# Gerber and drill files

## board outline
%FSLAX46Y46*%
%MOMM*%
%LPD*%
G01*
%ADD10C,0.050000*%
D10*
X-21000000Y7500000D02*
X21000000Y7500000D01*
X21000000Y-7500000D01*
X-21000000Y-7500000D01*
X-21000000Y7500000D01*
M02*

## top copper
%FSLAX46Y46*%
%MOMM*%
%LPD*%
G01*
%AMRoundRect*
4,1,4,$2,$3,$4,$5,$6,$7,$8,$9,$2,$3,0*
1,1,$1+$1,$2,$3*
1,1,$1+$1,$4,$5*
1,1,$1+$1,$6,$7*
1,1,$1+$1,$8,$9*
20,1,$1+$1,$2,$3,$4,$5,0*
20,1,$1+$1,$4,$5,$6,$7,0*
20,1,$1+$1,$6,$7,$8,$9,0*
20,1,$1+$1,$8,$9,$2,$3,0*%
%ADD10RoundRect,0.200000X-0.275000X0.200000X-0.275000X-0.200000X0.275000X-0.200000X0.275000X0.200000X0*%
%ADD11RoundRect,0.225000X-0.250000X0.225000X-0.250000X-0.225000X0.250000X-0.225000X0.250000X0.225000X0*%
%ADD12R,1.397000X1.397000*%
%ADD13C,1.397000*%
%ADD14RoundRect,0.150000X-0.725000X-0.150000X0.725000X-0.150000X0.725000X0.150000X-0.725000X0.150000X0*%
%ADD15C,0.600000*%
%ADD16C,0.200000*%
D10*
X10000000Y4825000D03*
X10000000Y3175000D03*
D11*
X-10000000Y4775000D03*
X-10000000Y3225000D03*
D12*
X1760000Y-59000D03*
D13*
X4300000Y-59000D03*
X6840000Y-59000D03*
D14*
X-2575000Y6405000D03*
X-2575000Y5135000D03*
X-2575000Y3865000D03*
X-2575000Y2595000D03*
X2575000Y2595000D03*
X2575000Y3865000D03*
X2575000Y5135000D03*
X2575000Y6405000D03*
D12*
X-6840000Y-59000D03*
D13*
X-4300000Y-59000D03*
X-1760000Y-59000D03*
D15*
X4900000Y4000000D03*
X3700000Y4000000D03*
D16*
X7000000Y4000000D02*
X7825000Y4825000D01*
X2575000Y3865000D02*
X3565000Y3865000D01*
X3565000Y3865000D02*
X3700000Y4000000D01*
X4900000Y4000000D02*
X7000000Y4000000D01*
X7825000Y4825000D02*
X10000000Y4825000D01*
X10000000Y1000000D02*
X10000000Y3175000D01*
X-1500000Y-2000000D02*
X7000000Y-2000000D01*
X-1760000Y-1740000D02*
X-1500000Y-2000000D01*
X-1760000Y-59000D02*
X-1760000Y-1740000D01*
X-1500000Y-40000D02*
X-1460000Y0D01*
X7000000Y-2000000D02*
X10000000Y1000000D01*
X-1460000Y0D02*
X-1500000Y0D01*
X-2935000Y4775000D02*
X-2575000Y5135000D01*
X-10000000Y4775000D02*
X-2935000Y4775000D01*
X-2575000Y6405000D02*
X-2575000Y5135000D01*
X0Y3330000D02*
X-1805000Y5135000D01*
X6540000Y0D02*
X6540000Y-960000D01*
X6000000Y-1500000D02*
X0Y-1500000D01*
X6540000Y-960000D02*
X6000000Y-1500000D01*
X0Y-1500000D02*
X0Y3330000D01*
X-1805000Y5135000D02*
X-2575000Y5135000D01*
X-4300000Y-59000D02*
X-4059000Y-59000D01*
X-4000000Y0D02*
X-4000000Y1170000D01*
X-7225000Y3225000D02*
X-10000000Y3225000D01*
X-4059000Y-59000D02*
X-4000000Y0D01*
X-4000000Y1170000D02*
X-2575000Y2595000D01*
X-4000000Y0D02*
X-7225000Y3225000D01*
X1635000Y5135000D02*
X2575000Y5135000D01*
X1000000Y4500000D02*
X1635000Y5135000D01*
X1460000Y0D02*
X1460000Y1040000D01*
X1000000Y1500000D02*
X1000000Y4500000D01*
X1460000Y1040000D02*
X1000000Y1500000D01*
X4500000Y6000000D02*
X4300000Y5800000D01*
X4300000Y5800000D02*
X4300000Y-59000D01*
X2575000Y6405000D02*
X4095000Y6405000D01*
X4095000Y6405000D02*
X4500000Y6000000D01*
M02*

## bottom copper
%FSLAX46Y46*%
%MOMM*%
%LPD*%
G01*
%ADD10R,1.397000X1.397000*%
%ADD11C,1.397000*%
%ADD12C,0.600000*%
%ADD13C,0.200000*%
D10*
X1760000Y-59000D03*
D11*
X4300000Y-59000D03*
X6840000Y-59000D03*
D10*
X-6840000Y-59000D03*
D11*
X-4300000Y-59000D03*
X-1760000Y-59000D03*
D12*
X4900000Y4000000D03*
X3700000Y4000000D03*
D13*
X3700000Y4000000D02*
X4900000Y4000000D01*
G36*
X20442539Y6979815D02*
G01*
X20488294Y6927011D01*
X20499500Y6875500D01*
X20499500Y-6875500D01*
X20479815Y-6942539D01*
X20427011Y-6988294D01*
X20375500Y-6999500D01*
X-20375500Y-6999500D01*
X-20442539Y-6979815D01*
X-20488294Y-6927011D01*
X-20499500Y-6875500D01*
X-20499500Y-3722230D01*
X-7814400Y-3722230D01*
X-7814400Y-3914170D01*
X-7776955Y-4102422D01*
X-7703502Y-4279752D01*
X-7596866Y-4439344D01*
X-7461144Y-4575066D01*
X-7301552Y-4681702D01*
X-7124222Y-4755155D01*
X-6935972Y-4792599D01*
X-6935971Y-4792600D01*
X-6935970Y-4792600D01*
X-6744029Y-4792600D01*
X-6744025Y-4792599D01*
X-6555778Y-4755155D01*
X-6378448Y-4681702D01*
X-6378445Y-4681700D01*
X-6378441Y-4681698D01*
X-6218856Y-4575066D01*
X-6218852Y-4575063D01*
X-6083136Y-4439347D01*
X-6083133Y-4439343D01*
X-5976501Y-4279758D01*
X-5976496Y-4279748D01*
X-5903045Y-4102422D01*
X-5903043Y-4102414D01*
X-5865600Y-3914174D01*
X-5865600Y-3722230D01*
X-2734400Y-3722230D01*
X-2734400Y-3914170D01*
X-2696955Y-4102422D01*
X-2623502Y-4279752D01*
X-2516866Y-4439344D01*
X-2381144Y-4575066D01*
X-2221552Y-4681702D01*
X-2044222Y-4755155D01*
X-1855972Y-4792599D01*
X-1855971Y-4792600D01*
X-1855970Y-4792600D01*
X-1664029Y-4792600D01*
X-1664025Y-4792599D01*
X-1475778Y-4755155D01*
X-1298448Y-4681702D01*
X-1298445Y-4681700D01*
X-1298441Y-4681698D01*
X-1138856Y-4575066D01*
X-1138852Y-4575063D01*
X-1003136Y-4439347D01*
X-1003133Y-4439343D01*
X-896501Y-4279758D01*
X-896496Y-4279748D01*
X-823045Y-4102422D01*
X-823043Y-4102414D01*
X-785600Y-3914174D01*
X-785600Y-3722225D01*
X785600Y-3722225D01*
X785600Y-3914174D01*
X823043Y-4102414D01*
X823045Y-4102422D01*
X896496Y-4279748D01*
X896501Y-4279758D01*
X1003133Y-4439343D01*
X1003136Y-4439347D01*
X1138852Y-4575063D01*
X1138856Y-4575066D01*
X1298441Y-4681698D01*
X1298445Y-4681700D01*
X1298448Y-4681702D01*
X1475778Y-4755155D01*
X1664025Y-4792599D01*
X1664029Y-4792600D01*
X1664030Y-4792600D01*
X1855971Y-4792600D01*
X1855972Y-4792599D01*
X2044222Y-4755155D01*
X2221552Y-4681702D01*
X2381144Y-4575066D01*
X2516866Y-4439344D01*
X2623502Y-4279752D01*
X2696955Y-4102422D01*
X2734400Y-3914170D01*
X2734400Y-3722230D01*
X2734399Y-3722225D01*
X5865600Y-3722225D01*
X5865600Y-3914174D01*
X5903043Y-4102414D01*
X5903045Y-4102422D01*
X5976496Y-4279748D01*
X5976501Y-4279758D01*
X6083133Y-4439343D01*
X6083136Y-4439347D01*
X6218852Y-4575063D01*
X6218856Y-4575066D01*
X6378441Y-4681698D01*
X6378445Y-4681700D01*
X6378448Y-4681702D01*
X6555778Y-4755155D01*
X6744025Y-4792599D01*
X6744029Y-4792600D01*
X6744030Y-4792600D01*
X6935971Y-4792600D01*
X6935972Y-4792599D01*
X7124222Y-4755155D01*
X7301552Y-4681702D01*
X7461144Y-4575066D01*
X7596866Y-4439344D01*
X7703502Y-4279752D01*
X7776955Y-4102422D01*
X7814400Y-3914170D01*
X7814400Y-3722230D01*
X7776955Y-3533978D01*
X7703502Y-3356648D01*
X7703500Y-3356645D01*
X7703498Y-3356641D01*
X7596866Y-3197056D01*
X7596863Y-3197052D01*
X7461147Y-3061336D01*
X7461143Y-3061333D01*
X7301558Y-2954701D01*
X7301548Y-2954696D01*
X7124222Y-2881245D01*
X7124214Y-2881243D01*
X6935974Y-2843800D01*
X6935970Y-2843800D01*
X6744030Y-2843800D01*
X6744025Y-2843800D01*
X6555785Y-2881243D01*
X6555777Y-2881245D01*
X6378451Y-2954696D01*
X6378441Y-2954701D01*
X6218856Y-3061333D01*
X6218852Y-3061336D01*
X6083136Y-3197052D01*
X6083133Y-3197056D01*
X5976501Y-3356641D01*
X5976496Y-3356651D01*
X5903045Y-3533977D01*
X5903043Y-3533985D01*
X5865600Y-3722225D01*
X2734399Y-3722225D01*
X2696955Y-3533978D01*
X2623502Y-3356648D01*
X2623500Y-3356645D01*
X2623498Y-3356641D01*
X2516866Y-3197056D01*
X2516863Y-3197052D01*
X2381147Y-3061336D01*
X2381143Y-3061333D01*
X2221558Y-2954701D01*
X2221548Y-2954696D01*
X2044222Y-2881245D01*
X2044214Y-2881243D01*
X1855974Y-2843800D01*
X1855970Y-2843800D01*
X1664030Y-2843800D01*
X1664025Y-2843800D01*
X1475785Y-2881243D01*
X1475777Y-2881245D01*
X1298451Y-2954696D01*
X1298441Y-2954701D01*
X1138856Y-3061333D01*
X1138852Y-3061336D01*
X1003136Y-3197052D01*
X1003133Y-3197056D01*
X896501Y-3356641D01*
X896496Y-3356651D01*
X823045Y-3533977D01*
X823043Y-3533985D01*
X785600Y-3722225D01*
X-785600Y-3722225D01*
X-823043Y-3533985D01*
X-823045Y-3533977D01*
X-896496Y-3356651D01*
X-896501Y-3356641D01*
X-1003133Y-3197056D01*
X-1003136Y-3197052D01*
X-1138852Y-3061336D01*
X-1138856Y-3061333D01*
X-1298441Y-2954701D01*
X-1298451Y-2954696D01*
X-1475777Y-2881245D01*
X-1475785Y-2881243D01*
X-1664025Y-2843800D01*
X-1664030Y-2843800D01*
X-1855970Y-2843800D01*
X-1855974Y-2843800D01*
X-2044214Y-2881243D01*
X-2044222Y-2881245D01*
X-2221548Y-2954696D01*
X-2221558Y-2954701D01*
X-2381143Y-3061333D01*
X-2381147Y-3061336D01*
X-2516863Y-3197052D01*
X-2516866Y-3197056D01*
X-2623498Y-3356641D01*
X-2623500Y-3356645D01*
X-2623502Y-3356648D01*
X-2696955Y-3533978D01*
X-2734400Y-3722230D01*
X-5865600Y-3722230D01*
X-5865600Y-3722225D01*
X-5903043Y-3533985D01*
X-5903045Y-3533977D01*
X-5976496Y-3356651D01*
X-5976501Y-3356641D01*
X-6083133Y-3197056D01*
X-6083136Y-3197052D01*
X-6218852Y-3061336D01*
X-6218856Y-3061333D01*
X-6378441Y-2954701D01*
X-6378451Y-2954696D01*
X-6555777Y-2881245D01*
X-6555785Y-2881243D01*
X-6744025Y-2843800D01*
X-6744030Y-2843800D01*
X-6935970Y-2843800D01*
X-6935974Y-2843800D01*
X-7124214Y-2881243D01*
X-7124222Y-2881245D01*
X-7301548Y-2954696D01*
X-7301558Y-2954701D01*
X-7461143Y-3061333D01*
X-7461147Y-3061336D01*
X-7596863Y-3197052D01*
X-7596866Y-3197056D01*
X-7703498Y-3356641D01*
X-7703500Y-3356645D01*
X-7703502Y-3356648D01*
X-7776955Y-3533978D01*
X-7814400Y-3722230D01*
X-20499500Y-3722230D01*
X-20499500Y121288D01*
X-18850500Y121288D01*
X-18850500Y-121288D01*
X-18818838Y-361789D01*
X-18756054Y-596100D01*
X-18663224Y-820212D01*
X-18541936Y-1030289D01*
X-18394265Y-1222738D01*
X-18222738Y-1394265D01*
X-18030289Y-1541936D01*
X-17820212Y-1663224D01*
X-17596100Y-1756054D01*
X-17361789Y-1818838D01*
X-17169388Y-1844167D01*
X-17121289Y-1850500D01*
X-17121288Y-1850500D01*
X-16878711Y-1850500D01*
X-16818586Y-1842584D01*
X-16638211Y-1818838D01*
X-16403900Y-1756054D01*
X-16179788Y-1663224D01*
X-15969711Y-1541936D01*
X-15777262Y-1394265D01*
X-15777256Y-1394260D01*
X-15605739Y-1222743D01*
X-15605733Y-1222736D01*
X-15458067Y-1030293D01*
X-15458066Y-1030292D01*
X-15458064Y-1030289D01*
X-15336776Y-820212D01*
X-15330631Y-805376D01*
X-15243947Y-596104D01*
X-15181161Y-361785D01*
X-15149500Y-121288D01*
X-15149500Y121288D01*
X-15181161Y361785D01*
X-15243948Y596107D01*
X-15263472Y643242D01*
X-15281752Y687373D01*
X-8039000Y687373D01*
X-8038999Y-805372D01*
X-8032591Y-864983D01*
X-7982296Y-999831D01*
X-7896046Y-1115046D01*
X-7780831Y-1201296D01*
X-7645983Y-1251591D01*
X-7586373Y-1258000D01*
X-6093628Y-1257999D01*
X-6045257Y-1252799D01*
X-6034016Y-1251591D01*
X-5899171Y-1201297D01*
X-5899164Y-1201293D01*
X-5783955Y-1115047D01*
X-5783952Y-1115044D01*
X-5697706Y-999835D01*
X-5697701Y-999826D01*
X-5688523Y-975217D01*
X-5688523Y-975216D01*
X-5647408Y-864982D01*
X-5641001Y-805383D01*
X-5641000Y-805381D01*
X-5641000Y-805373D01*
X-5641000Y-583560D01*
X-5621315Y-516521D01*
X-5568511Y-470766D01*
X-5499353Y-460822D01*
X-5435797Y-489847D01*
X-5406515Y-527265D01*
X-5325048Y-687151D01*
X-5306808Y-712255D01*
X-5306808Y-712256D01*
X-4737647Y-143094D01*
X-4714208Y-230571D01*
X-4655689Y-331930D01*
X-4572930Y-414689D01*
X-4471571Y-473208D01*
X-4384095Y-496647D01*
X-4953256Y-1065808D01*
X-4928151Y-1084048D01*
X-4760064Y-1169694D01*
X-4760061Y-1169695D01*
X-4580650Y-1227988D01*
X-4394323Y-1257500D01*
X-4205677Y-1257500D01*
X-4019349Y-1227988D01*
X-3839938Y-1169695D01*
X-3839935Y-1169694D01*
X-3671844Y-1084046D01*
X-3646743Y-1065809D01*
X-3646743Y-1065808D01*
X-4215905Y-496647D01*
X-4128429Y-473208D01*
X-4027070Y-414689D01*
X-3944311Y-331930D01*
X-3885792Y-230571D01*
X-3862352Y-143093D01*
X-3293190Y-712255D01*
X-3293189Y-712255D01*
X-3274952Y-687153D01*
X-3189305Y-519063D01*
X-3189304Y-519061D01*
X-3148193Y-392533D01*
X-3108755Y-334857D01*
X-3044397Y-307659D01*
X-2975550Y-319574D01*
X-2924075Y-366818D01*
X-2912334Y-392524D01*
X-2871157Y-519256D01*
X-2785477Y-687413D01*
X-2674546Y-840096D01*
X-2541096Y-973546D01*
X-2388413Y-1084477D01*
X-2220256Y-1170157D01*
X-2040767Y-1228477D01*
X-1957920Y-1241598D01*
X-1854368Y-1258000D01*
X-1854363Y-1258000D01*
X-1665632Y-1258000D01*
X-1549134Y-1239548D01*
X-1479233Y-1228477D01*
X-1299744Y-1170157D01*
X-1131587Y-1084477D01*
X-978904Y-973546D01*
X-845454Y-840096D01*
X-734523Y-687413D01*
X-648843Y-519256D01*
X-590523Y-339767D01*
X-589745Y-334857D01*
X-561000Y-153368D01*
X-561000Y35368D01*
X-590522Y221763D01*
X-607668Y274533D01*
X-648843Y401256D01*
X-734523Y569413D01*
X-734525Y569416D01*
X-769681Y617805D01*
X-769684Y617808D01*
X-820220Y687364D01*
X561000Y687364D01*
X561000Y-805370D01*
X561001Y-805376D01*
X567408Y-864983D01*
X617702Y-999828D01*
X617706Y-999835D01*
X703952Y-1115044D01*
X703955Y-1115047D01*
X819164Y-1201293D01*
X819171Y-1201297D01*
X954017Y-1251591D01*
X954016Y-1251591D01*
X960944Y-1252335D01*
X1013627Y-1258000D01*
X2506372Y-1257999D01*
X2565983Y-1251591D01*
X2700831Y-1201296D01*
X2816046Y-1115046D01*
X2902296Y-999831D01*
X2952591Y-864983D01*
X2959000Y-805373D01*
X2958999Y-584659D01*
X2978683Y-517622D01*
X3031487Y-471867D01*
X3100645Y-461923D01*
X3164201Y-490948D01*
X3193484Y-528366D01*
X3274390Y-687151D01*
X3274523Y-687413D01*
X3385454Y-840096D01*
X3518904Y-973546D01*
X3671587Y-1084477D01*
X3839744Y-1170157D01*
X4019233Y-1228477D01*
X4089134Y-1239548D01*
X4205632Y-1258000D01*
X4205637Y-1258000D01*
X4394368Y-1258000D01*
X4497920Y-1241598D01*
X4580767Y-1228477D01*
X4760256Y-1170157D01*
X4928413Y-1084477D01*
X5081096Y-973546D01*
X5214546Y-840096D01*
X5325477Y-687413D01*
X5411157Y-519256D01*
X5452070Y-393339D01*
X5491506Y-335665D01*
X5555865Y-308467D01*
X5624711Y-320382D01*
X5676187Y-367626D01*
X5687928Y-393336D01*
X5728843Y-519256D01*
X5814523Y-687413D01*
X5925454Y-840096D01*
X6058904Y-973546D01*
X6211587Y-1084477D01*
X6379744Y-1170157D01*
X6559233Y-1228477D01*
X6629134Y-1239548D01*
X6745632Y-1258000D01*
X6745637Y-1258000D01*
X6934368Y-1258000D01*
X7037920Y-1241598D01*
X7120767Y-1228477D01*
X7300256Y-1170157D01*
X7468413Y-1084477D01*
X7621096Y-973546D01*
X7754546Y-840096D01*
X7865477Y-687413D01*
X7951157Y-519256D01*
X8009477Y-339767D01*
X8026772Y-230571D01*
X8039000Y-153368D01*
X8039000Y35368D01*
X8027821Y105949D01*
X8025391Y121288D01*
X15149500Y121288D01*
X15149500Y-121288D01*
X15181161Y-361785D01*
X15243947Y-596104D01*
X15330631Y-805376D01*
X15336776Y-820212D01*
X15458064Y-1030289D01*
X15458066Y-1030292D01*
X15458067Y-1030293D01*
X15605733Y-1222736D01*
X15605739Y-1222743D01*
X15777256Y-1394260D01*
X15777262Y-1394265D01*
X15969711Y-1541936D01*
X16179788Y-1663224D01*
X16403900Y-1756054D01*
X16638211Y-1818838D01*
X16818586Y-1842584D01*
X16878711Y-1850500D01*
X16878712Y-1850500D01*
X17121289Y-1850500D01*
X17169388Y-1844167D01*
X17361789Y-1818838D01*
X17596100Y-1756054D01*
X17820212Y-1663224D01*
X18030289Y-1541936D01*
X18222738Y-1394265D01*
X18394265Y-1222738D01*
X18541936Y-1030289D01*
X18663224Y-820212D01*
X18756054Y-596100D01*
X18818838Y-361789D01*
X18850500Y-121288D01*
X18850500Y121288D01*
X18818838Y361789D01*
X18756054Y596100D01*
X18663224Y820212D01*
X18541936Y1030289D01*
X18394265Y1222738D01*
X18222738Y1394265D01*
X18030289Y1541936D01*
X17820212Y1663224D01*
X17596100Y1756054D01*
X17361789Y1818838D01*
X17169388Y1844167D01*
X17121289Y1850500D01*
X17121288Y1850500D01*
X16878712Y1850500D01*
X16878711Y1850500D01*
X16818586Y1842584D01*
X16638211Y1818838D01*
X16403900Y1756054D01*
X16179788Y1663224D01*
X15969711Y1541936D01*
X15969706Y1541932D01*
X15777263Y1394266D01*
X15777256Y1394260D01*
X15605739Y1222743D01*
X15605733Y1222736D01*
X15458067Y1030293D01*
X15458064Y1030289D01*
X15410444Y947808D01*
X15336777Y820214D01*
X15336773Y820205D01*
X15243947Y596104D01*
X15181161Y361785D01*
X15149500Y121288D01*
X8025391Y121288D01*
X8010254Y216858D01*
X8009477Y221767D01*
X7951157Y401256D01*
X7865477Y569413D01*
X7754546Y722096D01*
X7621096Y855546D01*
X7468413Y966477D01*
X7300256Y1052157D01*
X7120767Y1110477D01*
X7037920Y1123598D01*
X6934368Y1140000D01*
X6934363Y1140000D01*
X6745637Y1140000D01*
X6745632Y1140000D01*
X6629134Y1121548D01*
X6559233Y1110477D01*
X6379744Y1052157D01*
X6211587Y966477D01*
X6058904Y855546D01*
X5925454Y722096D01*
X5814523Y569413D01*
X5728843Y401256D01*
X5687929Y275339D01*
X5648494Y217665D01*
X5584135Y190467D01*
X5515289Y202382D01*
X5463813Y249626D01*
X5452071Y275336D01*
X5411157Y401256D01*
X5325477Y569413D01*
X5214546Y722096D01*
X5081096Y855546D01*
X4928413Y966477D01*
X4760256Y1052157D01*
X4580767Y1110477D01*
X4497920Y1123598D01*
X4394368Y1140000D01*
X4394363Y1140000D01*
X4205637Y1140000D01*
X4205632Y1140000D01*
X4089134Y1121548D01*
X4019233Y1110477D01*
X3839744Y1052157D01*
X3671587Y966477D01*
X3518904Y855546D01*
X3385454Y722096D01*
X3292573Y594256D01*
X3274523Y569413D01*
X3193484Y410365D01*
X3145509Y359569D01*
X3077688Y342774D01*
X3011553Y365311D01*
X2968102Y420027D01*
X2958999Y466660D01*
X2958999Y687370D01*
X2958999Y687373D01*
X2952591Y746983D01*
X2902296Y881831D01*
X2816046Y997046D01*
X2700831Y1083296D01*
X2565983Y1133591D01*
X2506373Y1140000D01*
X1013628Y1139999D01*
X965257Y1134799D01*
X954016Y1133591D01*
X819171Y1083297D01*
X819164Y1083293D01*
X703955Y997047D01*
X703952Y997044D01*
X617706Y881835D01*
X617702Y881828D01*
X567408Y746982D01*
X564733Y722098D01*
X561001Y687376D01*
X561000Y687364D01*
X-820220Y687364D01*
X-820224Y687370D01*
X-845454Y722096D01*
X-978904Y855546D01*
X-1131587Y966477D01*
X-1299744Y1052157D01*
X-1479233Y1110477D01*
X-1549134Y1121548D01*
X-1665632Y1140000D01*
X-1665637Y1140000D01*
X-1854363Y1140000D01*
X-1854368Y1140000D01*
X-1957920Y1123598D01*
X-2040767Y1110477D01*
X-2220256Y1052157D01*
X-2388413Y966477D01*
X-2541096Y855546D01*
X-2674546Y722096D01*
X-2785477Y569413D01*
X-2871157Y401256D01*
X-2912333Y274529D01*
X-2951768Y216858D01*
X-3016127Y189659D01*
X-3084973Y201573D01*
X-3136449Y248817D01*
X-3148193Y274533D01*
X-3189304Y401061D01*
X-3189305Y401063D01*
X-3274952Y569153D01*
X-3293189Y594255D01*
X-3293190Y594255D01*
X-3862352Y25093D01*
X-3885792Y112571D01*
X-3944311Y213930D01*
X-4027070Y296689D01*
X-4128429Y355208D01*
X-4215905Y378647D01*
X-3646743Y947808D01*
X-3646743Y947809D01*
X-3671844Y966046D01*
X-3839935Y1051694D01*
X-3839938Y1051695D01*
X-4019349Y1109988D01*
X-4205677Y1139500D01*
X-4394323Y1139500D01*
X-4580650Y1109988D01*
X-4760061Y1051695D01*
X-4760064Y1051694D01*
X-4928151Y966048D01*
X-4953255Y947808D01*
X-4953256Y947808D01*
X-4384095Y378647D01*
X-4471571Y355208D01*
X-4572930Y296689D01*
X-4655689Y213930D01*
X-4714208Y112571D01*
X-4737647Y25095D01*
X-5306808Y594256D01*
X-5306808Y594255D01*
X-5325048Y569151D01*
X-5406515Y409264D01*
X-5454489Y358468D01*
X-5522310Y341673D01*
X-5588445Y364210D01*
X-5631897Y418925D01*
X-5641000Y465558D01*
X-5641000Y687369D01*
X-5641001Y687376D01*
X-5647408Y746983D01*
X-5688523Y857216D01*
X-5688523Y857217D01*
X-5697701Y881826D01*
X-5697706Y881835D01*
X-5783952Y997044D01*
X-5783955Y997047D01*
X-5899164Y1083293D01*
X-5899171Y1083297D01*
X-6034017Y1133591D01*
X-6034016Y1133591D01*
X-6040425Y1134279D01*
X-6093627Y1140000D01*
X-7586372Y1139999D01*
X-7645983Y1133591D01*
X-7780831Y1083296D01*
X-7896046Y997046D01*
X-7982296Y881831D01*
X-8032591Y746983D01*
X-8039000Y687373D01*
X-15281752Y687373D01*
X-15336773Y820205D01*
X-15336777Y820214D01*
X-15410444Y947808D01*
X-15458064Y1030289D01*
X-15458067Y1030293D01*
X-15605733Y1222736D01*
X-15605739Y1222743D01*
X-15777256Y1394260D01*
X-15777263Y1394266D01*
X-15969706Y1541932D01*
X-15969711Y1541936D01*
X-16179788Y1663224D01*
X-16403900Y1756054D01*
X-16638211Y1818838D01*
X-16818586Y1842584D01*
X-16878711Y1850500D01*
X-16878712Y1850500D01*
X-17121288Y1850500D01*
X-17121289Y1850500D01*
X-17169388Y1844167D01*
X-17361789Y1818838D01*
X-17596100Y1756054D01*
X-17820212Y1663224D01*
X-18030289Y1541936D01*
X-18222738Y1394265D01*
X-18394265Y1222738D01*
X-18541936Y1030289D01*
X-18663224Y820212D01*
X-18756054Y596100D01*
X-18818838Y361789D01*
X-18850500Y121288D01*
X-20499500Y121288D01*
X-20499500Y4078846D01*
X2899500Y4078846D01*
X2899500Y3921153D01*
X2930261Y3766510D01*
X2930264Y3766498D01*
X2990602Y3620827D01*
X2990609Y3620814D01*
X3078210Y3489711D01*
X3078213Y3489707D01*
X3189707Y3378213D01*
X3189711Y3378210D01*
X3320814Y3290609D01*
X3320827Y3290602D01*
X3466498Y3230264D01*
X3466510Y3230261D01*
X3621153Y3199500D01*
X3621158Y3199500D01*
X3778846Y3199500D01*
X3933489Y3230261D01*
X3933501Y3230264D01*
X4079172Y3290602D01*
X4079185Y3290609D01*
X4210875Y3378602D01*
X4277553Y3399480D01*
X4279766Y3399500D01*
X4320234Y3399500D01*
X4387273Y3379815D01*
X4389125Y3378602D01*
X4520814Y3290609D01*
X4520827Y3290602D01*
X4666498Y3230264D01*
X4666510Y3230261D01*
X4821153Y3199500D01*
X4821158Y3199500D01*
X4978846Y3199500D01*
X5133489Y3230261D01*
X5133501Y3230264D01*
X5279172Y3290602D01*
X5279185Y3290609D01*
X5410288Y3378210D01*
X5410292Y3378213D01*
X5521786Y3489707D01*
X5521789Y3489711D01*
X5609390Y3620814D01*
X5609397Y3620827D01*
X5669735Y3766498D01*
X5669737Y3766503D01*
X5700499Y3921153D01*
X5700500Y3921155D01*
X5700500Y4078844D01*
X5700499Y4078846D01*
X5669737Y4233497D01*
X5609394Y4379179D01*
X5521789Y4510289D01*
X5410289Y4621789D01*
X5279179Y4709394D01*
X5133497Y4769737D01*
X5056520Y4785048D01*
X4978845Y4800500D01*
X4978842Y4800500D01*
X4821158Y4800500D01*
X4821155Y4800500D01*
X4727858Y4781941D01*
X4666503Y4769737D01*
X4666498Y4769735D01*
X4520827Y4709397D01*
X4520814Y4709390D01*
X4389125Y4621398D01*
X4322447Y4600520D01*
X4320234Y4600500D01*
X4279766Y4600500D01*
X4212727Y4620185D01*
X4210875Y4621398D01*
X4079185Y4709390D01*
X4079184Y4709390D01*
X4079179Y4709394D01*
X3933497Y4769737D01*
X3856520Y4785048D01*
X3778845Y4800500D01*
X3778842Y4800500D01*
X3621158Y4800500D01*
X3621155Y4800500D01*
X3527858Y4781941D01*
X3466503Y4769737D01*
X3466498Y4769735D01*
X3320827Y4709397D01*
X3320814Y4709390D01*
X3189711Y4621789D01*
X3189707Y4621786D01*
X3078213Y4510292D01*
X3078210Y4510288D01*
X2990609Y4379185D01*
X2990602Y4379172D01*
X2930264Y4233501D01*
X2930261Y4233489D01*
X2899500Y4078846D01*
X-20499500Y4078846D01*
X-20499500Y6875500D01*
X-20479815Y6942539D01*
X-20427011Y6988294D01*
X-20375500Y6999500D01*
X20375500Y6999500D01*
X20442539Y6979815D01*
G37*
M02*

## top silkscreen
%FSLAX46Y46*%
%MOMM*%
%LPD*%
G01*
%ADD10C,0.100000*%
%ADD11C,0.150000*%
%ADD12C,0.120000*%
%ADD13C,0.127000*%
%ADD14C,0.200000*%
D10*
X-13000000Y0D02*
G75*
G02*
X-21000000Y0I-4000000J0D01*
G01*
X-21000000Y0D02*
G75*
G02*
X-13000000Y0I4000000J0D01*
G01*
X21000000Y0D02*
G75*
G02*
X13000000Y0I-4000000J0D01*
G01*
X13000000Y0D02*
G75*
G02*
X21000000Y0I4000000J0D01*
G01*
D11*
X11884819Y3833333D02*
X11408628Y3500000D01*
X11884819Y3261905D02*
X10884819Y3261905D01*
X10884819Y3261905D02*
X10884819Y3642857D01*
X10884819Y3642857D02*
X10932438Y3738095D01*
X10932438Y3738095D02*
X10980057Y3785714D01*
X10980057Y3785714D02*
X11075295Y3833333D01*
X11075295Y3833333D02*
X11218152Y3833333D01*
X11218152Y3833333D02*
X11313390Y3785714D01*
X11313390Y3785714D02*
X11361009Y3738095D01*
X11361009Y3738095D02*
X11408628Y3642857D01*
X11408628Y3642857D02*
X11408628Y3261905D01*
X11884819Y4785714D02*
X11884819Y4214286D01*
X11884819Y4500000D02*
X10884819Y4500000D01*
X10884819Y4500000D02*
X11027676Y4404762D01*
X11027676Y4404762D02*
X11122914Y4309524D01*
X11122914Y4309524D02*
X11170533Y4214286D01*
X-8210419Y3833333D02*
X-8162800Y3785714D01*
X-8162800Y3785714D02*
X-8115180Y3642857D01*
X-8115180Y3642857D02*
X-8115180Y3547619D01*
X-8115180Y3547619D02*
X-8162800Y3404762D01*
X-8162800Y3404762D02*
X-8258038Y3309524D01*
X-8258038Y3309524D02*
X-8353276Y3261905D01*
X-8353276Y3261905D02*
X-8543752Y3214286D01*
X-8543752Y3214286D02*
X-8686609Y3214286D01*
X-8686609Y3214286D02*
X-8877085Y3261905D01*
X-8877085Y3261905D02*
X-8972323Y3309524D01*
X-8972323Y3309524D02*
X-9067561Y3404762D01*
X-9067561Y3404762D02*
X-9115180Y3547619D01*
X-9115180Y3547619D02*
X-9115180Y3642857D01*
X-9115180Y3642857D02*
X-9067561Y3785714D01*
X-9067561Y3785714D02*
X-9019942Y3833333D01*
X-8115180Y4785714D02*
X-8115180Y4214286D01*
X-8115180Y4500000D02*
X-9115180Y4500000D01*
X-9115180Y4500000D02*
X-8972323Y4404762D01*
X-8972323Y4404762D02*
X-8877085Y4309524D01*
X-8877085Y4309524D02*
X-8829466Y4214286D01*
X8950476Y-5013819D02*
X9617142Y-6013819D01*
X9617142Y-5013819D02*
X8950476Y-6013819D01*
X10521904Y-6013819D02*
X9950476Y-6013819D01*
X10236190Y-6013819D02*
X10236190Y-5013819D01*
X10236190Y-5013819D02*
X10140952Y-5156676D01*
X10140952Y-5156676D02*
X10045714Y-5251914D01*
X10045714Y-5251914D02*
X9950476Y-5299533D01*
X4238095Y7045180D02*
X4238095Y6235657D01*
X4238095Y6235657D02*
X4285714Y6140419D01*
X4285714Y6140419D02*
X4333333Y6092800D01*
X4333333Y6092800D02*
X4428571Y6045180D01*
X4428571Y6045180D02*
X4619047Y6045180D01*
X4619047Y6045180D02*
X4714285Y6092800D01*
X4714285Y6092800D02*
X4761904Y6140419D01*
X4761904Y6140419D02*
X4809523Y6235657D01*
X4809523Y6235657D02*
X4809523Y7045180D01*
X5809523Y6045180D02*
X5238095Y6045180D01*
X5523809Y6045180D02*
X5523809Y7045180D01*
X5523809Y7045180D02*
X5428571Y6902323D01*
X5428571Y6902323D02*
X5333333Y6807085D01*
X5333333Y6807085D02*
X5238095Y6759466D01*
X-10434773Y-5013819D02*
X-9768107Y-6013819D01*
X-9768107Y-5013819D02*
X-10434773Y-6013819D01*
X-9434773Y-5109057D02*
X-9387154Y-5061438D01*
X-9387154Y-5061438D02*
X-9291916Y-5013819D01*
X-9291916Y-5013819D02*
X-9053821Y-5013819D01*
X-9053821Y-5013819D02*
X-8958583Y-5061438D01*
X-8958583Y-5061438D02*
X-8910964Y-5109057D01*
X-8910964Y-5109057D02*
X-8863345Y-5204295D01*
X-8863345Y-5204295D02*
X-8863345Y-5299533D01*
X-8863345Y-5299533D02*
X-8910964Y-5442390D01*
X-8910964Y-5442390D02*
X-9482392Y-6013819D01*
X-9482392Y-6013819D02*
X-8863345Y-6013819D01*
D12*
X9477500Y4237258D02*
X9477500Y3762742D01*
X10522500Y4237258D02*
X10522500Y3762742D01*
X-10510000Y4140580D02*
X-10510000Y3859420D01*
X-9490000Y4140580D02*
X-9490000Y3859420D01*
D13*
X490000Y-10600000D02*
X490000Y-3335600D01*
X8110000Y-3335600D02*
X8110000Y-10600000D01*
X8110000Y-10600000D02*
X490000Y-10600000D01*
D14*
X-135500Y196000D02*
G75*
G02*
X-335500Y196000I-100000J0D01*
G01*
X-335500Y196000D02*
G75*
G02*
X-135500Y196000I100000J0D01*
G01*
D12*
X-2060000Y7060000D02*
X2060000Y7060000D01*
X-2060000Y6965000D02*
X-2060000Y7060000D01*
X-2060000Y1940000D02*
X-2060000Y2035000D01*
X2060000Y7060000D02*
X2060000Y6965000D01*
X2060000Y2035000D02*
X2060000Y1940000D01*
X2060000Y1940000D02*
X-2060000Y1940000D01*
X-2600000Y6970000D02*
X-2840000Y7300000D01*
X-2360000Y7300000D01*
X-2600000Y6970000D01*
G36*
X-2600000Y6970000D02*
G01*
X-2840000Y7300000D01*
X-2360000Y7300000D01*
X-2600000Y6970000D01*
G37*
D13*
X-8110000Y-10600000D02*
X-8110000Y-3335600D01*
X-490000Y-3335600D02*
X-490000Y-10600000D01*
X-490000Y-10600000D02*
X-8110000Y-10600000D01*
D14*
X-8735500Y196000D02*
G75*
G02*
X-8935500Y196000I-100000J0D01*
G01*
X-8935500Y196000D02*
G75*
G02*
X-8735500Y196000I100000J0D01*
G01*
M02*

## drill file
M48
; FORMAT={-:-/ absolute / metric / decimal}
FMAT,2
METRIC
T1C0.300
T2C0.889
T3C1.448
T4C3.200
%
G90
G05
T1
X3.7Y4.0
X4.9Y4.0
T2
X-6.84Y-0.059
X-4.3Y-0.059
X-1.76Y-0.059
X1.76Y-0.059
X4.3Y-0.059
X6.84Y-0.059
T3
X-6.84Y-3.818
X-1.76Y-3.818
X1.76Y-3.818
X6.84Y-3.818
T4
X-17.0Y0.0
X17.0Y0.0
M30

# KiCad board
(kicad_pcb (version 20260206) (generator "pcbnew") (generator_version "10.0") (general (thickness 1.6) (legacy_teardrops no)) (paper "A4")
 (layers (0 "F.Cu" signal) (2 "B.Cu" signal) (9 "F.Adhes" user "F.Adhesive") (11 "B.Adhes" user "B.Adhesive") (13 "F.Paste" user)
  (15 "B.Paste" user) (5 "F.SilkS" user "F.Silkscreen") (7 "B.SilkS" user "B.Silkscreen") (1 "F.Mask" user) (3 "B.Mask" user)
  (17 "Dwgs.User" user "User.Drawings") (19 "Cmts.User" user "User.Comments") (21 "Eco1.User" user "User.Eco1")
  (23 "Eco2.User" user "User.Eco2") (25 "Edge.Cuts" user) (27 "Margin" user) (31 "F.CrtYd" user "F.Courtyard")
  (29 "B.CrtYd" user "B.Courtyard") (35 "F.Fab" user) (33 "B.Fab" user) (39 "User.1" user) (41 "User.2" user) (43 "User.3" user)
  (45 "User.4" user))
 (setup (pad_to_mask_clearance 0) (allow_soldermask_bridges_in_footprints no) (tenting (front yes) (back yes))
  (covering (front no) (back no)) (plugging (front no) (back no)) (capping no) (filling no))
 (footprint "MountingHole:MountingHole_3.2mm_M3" (layer "F.Cu") (at 17 0)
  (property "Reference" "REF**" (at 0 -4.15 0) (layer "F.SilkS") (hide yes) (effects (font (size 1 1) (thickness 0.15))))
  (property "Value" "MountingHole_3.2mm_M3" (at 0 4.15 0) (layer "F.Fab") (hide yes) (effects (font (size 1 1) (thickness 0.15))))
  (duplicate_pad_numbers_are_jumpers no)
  (pad "" np_thru_hole circle (at 0 0) (size 3.2 3.2) (drill 3.2) (layers "*.Cu" "*.Mask")))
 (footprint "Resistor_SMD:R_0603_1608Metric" (layer "F.Cu") (at 10 -4 -90)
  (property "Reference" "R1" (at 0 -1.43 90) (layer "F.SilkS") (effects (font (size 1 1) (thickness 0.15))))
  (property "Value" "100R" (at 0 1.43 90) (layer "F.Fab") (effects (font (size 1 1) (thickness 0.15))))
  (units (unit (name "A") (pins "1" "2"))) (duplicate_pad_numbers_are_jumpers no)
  (fp_line (start -0.237258 0.5225) (end 0.237258 0.5225) (stroke (width 0.12) (type solid)) (layer "F.SilkS"))
  (fp_line (start -0.237258 -0.5225) (end 0.237258 -0.5225) (stroke (width 0.12) (type solid)) (layer "F.SilkS"))
  (pad "1" smd roundrect (at -0.825 0 270) (size 0.8 0.95) (layers "F.Cu" "F.Mask" "F.Paste") (roundrect_rratio 0.25) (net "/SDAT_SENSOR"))
  (pad "2" smd roundrect (at 0.825 0 270) (size 0.8 0.95) (layers "F.Cu" "F.Mask" "F.Paste") (roundrect_rratio 0.25) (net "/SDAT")))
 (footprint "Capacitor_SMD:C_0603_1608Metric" (layer "F.Cu") (at -10 -4 -90)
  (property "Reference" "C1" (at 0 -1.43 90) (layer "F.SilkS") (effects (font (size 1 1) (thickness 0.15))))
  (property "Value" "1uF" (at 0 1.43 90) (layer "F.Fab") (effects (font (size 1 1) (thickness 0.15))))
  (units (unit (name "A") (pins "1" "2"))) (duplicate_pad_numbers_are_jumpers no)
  (fp_line (start -0.14058 0.51) (end 0.14058 0.51) (stroke (width 0.12) (type solid)) (layer "F.SilkS"))
  (fp_line (start -0.14058 -0.51) (end 0.14058 -0.51) (stroke (width 0.12) (type solid)) (layer "F.SilkS"))
  (pad "1" smd roundrect (at -0.775 0 270) (size 0.9 0.95) (layers "F.Cu" "F.Mask" "F.Paste") (roundrect_rratio 0.25) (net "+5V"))
  (pad "2" smd roundrect (at 0.775 0 270) (size 0.9 0.95) (layers "F.Cu" "F.Mask" "F.Paste") (roundrect_rratio 0.25) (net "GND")))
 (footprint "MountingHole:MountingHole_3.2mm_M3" (layer "F.Cu") (at -17 0)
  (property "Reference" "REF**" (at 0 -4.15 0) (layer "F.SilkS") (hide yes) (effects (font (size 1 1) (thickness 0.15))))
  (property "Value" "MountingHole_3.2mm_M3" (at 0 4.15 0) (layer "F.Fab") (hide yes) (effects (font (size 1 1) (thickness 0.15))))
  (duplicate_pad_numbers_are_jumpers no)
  (pad "" np_thru_hole circle (at 0 0) (size 3.2 3.2) (drill 3.2) (layers "*.Cu" "*.Mask")))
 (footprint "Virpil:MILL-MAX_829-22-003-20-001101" (layer "F.Cu") (at 4.3 0.059)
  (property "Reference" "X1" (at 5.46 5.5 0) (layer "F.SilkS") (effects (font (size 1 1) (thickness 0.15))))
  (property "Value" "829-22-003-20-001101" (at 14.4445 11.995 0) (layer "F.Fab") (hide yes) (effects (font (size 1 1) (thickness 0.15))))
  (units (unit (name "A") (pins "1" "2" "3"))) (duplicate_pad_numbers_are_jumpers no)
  (fp_line (start -3.81 10.541) (end -3.81 3.2766) (stroke (width 0.127) (type solid)) (layer "F.SilkS"))
  (fp_line (start 3.81 3.2766) (end 3.81 10.541) (stroke (width 0.127) (type solid)) (layer "F.SilkS"))
  (fp_line (start 3.81 10.541) (end -3.81 10.541) (stroke (width 0.127) (type solid)) (layer "F.SilkS"))
  (fp_circle (center -4.5355 -0.255) (end -4.4355 -0.255) (stroke (width 0.2) (type solid)) (fill no) (layer "F.SilkS"))
  (pad "" np_thru_hole circle (at -2.54 3.7592) (size 1.4478 1.4478) (drill 1.4478) (layers "*.Cu" "*.Mask"))
  (pad "" np_thru_hole circle (at 2.54 3.7592) (size 1.4478 1.4478) (drill 1.4478) (layers "*.Cu" "*.Mask"))
  (pad "1" thru_hole rect (at -2.54 0) (size 1.397 1.397) (drill 0.889) (layers "*.Cu" "*.Mask") (remove_unused_layers no) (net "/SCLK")
   (solder_mask_margin 0.102))
  (pad "2" thru_hole circle (at 0 0) (size 1.397 1.397) (drill 0.889) (layers "*.Cu" "*.Mask") (remove_unused_layers no) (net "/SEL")
   (solder_mask_margin 0.102))
  (pad "3" thru_hole circle (at 2.54 0) (size 1.397 1.397) (drill 0.889) (layers "*.Cu" "*.Mask") (remove_unused_layers no) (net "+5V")
   (solder_mask_margin 0.102)))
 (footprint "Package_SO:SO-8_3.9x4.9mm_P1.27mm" (layer "F.Cu") (at 0 -4.5)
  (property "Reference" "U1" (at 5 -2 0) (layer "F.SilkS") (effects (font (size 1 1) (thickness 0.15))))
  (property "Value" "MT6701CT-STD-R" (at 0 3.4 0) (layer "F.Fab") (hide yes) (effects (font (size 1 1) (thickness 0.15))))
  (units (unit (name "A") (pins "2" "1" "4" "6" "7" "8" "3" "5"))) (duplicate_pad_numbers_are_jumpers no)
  (fp_line (start -2.06 -2.56) (end 2.06 -2.56) (stroke (width 0.12) (type solid)) (layer "F.SilkS"))
  (fp_line (start -2.06 -2.465) (end -2.06 -2.56) (stroke (width 0.12) (type solid)) (layer "F.SilkS"))
  (fp_line (start -2.06 2.56) (end -2.06 2.465) (stroke (width 0.12) (type solid)) (layer "F.SilkS"))
  (fp_line (start 2.06 -2.56) (end 2.06 -2.465) (stroke (width 0.12) (type solid)) (layer "F.SilkS"))
  (fp_line (start 2.06 2.465) (end 2.06 2.56) (stroke (width 0.12) (type solid)) (layer "F.SilkS"))
  (fp_line (start 2.06 2.56) (end -2.06 2.56) (stroke (width 0.12) (type solid)) (layer "F.SilkS"))
  (fp_poly (pts (xy -2.6 -2.47) (xy -2.84 -2.8) (xy -2.36 -2.8)) (stroke (width 0.12) (type solid)) (fill yes) (layer "F.SilkS"))
  (pad "1" smd roundrect (at -2.575 -1.905) (size 1.75 0.6) (layers "F.Cu" "F.Mask" "F.Paste") (roundrect_rratio 0.25) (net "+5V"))
  (pad "2" smd roundrect (at -2.575 -0.635) (size 1.75 0.6) (layers "F.Cu" "F.Mask" "F.Paste") (roundrect_rratio 0.25) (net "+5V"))
  (pad "3" smd roundrect (at -2.575 0.635) (size 1.75 0.6) (layers "F.Cu" "F.Mask" "F.Paste") (roundrect_rratio 0.25)
   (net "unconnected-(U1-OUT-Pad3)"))
  (pad "4" smd roundrect (at -2.575 1.905) (size 1.75 0.6) (layers "F.Cu" "F.Mask" "F.Paste") (roundrect_rratio 0.25) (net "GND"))
  (pad "5" smd roundrect (at 2.575 1.905) (size 1.75 0.6) (layers "F.Cu" "F.Mask" "F.Paste") (roundrect_rratio 0.25)
   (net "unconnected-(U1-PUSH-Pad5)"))
  (pad "6" smd roundrect (at 2.575 0.635) (size 1.75 0.6) (layers "F.Cu" "F.Mask" "F.Paste") (roundrect_rratio 0.25) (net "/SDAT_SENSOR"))
  (pad "7" smd roundrect (at 2.575 -0.635) (size 1.75 0.6) (layers "F.Cu" "F.Mask" "F.Paste") (roundrect_rratio 0.25) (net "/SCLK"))
  (pad "8" smd roundrect (at 2.575 -1.905) (size 1.75 0.6) (layers "F.Cu" "F.Mask" "F.Paste") (roundrect_rratio 0.25) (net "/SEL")))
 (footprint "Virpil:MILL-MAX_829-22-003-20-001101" (layer "F.Cu") (at -4.3 0.059)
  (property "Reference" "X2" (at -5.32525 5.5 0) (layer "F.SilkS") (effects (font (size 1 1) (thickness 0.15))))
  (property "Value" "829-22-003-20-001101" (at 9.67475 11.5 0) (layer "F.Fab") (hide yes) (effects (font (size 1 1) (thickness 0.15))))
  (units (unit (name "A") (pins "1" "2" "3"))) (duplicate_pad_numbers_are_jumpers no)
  (fp_line (start -3.81 10.541) (end -3.81 3.2766) (stroke (width 0.127) (type solid)) (layer "F.SilkS"))
  (fp_line (start 3.81 3.2766) (end 3.81 10.541) (stroke (width 0.127) (type solid)) (layer "F.SilkS"))
  (fp_line (start 3.81 10.541) (end -3.81 10.541) (stroke (width 0.127) (type solid)) (layer "F.SilkS"))
  (fp_circle (center -4.5355 -0.255) (end -4.4355 -0.255) (stroke (width 0.2) (type solid)) (fill no) (layer "F.SilkS"))
  (pad "" np_thru_hole circle (at -2.54 3.7592) (size 1.4478 1.4478) (drill 1.4478) (layers "*.Cu" "*.Mask"))
  (pad "" np_thru_hole circle (at 2.54 3.7592) (size 1.4478 1.4478) (drill 1.4478) (layers "*.Cu" "*.Mask"))
  (pad "1" thru_hole rect (at -2.54 0) (size 1.397 1.397) (drill 0.889) (layers "*.Cu" "*.Mask") (remove_unused_layers no) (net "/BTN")
   (solder_mask_margin 0.102))
  (pad "2" thru_hole circle (at 0 0) (size 1.397 1.397) (drill 0.889) (layers "*.Cu" "*.Mask") (remove_unused_layers no) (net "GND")
   (solder_mask_margin 0.102))
  (pad "3" thru_hole circle (at 2.54 0) (size 1.397 1.397) (drill 0.889) (layers "*.Cu" "*.Mask") (remove_unused_layers no) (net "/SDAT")
   (solder_mask_margin 0.102)))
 (gr_circle (center -17 0) (end -13 0) (stroke (width 0.1) (type default)) (fill no) (layer "F.SilkS"))
 (gr_circle (center 17 0) (end 21 0) (stroke (width 0.1) (type default)) (fill no) (layer "F.SilkS"))
 (gr_rect (start -21 -7.5) (end 21 7.5) (stroke (width 0.05) (type default)) (fill no) (layer "Edge.Cuts"))
 (segment (start 7 -4) (end 7.825 -4.825) (width 0.2) (layer "F.Cu") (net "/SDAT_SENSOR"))
 (segment (start 2.575 -3.865) (end 3.565 -3.865) (width 0.2) (layer "F.Cu") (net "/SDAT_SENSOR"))
 (segment (start 3.565 -3.865) (end 3.7 -4) (width 0.2) (layer "F.Cu") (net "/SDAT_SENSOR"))
 (segment (start 4.9 -4) (end 7 -4) (width 0.2) (layer "F.Cu") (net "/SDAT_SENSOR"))
 (segment (start 7.825 -4.825) (end 10 -4.825) (width 0.2) (layer "F.Cu") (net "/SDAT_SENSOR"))
 (via (at 4.9 -4) (size 0.6) (drill 0.3) (layers "F.Cu" "B.Cu") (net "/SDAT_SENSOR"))
 (via (at 3.7 -4) (size 0.6) (drill 0.3) (layers "F.Cu" "B.Cu") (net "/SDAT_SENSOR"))
 (segment (start 3.7 -4) (end 4.9 -4) (width 0.2) (layer "B.Cu") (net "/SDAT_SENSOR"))
 (segment (start 10 -1) (end 10 -3.175) (width 0.2) (layer "F.Cu") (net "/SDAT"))
 (segment (start -1.5 2) (end 7 2) (width 0.2) (layer "F.Cu") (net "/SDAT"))
 (segment (start -1.76 1.74) (end -1.5 2) (width 0.2) (layer "F.Cu") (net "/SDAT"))
 (segment (start -1.76 0.059) (end -1.76 1.74) (width 0.2) (layer "F.Cu") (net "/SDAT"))
 (segment (start -1.5 0.04) (end -1.46 0) (width 0.2) (layer "F.Cu") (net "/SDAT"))
 (segment (start 7 2) (end 10 -1) (width 0.2) (layer "F.Cu") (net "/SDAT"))
 (segment (start -1.46 0) (end -1.5 0) (width 0.2) (layer "F.Cu") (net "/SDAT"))
 (segment (start -2.935 -4.775) (end -2.575 -5.135) (width 0.2) (layer "F.Cu") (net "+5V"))
 (segment (start -10 -4.775) (end -2.935 -4.775) (width 0.2) (layer "F.Cu") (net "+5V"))
 (segment (start -2.575 -6.405) (end -2.575 -5.135) (width 0.2) (layer "F.Cu") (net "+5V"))
 (segment (start 0 -3.33) (end -1.805 -5.135) (width 0.2) (layer "F.Cu") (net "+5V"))
 (segment (start 6.54 0) (end 6.54 0.96) (width 0.2) (layer "F.Cu") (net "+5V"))
 (segment (start 6 1.5) (end 0 1.5) (width 0.2) (layer "F.Cu") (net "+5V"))
 (segment (start 6.54 0.96) (end 6 1.5) (width 0.2) (layer "F.Cu") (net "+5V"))
 (segment (start 0 1.5) (end 0 -3.33) (width 0.2) (layer "F.Cu") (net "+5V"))
 (segment (start -1.805 -5.135) (end -2.575 -5.135) (width 0.2) (layer "F.Cu") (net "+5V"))
 (segment (start -4.3 0.059) (end -4.059 0.059) (width 0.2) (layer "F.Cu") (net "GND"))
 (segment (start -4 0) (end -4 -1.17) (width 0.2) (layer "F.Cu") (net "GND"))
 (segment (start -7.225 -3.225) (end -10 -3.225) (width 0.2) (layer "F.Cu") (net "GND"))
 (segment (start -4.059 0.059) (end -4 0) (width 0.2) (layer "F.Cu") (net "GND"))
 (segment (start -4 -1.17) (end -2.575 -2.595) (width 0.2) (layer "F.Cu") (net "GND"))
 (segment (start -4 0) (end -7.225 -3.225) (width 0.2) (layer "F.Cu") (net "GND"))
 (segment (start 1.635 -5.135) (end 2.575 -5.135) (width 0.2) (layer "F.Cu") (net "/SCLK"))
 (segment (start 1 -4.5) (end 1.635 -5.135) (width 0.2) (layer "F.Cu") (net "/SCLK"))
 (segment (start 1.46 0) (end 1.46 -1.04) (width 0.2) (layer "F.Cu") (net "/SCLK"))
 (segment (start 1 -1.5) (end 1 -4.5) (width 0.2) (layer "F.Cu") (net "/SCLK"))
 (segment (start 1.46 -1.04) (end 1 -1.5) (width 0.2) (layer "F.Cu") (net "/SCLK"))
 (segment (start 4.5 -6) (end 4.3 -5.8) (width 0.2) (layer "F.Cu") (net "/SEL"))
 (segment (start 4.3 -5.8) (end 4.3 0.059) (width 0.2) (layer "F.Cu") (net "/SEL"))
 (segment (start 2.575 -6.405) (end 4.095 -6.405) (width 0.2) (layer "F.Cu") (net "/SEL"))
 (segment (start 4.095 -6.405) (end 4.5 -6) (width 0.2) (layer "F.Cu") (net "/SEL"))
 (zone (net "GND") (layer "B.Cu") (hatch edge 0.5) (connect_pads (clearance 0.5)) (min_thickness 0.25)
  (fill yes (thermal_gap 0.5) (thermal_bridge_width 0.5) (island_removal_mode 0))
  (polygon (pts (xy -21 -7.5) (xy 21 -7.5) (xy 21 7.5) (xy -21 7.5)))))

